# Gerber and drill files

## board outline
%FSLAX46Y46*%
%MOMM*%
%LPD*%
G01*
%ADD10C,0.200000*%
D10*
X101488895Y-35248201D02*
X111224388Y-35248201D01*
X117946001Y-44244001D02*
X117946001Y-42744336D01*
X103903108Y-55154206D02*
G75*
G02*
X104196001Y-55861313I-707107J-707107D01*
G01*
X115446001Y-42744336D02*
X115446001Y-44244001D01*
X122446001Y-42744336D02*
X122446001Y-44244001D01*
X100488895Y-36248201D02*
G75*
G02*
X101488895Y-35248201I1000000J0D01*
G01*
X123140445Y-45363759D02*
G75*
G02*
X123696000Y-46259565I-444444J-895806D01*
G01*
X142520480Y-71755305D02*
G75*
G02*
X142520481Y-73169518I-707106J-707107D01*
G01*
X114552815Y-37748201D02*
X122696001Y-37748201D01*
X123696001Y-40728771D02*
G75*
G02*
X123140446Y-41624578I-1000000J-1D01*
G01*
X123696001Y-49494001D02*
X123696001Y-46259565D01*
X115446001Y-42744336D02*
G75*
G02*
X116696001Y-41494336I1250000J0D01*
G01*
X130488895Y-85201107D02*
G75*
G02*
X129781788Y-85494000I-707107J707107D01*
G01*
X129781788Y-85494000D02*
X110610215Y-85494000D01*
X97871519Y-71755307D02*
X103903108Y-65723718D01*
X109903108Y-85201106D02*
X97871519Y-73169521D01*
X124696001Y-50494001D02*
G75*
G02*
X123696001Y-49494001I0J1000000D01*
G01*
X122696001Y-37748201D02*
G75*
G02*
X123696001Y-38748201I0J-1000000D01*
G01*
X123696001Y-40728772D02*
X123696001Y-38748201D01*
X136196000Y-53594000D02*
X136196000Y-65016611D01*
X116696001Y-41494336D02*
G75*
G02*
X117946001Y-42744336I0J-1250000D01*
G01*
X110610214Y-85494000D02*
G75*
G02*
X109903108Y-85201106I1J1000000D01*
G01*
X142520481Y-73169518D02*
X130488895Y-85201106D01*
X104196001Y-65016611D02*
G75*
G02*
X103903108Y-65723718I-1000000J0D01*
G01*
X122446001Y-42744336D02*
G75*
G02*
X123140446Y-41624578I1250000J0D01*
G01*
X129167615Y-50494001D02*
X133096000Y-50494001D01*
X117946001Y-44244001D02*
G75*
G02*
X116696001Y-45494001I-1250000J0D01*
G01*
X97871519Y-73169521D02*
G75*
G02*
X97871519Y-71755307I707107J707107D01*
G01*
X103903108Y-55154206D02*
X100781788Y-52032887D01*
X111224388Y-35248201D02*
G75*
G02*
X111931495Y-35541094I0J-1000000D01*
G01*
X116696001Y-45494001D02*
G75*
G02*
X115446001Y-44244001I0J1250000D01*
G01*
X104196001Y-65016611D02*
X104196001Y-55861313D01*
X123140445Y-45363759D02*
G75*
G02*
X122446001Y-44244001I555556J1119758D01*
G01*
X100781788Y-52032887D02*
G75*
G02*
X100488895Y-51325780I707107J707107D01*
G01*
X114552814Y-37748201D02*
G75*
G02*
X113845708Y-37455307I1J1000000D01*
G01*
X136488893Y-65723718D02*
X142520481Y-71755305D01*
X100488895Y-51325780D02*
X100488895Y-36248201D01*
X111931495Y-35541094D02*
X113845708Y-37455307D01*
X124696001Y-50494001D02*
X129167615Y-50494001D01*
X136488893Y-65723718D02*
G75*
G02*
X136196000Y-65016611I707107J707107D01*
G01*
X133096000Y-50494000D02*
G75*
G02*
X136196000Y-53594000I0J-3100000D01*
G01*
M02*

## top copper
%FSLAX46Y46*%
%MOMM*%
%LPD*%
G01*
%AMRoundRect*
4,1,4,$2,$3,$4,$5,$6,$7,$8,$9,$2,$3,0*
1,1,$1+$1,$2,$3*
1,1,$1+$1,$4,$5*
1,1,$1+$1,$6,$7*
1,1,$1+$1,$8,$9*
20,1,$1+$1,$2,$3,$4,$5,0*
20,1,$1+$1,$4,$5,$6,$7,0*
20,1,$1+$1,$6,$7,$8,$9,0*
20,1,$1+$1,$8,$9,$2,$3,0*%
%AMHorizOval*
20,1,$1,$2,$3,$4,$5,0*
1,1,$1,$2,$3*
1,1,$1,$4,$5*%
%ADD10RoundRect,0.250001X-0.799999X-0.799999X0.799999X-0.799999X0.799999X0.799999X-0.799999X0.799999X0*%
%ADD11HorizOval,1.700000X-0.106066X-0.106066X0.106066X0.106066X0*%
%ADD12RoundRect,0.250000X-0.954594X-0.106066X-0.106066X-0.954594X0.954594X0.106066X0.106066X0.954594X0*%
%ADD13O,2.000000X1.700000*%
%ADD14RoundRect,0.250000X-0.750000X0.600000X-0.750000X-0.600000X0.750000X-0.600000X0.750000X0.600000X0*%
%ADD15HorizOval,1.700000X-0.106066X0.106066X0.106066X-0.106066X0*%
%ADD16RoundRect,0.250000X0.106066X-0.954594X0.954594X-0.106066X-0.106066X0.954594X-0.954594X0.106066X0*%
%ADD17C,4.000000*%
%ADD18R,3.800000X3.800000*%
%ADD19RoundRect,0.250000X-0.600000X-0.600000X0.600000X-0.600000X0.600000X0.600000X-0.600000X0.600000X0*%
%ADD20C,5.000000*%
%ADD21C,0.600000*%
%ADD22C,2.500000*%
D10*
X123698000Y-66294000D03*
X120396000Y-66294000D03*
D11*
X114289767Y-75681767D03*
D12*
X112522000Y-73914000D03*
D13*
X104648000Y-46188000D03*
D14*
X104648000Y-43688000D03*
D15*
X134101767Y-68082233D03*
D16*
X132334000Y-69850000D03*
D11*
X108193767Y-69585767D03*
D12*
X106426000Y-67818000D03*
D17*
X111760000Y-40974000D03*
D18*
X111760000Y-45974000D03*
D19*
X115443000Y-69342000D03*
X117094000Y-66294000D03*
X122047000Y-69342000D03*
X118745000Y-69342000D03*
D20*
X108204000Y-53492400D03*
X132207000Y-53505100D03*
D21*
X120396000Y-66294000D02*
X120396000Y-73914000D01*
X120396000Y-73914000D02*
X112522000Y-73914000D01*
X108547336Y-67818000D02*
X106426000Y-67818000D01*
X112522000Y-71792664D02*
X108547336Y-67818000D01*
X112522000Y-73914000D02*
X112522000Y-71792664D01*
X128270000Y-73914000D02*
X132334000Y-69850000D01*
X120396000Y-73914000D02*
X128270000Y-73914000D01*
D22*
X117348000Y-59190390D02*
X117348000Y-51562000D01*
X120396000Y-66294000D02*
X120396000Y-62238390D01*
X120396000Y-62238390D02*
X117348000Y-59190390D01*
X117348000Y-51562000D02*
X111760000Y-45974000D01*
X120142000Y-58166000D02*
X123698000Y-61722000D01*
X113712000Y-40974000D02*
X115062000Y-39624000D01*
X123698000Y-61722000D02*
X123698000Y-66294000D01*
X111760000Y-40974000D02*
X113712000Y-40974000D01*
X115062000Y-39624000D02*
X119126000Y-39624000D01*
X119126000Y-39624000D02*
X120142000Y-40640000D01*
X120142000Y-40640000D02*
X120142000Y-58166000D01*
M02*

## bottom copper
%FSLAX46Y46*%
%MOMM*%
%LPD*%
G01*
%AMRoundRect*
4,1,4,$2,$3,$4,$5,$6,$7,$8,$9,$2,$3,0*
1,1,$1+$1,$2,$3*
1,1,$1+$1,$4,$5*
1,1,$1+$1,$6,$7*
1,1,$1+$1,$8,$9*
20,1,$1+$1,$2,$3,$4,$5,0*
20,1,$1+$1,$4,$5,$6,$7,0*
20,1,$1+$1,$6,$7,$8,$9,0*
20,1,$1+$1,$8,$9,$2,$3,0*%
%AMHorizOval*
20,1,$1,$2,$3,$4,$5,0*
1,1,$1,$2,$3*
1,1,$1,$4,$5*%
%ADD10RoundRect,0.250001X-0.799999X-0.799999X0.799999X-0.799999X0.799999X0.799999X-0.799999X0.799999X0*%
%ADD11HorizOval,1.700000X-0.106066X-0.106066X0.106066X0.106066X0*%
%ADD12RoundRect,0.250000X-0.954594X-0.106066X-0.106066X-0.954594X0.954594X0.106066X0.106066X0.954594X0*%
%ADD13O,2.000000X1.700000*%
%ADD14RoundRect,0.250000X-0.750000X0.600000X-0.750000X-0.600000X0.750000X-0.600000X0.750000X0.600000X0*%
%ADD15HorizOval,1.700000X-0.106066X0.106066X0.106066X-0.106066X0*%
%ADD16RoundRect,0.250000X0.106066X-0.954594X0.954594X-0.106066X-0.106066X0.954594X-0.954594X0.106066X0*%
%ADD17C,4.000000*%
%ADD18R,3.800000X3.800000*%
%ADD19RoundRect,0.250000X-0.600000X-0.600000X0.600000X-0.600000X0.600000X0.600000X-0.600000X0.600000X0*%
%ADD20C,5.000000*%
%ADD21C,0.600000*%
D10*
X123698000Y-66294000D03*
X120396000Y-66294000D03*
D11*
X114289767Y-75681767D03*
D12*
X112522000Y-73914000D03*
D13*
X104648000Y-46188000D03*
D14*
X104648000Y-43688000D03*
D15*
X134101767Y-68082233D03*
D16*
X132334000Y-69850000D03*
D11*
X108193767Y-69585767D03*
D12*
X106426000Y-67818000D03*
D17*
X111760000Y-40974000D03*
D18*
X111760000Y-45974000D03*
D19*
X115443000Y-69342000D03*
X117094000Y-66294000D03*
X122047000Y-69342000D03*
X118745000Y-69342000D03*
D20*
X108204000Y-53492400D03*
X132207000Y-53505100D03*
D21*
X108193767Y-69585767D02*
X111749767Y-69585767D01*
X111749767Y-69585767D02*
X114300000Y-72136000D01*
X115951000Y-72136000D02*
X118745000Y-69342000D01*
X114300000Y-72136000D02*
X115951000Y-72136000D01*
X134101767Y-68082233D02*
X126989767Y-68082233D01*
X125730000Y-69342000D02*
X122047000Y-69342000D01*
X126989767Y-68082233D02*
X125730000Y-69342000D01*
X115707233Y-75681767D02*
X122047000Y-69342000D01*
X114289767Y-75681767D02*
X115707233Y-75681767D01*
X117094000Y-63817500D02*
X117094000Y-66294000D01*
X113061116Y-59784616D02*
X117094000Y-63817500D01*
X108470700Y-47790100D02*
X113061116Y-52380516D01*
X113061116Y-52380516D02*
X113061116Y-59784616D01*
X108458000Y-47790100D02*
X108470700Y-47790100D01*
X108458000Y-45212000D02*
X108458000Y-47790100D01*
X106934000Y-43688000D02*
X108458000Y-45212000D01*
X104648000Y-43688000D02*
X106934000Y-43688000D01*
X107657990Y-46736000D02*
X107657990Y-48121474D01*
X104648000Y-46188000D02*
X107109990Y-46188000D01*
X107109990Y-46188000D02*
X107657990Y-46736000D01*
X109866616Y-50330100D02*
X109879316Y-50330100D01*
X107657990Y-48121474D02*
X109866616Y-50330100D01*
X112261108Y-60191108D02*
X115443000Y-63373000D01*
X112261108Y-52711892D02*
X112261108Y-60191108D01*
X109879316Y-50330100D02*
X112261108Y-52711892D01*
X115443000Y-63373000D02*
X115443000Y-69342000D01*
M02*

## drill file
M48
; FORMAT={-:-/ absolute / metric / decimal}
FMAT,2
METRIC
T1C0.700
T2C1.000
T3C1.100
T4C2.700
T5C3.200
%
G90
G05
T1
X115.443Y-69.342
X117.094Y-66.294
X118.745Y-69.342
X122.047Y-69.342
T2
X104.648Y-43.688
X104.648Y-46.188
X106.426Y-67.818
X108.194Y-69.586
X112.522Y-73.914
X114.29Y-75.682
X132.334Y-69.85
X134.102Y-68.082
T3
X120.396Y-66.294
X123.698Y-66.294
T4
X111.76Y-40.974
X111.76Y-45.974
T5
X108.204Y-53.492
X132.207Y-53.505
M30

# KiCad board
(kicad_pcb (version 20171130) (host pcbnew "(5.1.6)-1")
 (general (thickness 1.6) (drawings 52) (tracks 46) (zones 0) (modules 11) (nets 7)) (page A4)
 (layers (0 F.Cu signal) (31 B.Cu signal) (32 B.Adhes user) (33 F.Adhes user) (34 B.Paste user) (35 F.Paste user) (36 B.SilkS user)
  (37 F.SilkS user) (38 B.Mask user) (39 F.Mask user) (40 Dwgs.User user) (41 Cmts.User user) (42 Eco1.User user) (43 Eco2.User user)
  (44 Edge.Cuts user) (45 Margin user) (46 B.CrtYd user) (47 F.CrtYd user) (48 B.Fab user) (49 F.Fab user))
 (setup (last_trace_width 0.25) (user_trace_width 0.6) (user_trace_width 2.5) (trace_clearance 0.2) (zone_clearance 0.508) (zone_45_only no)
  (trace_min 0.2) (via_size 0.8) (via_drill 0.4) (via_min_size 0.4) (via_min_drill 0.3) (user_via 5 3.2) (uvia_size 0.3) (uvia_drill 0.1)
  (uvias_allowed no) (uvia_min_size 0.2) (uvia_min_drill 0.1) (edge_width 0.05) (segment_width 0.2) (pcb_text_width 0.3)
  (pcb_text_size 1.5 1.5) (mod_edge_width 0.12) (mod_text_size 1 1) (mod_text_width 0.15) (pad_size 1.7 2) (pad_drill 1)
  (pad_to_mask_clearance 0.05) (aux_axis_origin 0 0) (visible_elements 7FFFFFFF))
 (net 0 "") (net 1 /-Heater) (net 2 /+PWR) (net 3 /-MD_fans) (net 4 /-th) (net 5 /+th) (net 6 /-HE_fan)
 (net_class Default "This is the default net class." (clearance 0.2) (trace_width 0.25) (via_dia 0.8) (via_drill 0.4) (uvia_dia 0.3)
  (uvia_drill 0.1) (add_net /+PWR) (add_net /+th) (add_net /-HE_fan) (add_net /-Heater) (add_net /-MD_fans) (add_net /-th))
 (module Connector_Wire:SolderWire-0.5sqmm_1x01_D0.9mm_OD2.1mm (layer F.Cu) (at 123.698 66.294)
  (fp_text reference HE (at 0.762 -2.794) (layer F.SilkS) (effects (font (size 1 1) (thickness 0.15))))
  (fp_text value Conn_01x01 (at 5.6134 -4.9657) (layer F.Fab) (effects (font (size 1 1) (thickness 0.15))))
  (pad 1 thru_hole roundrect (at 0 0) (size 2.1 2.1) (drill 1.1) (layers *.Cu *.Mask) (roundrect_rratio 0.119048) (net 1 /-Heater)))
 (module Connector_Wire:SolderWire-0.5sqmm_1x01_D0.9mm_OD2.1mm (layer F.Cu) (at 120.396 66.294)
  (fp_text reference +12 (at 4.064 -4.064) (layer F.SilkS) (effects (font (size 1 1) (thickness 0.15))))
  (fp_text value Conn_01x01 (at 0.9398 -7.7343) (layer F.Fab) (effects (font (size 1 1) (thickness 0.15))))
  (pad 1 thru_hole roundrect (at 0 0) (size 2.1 2.1) (drill 1.1) (layers *.Cu *.Mask) (roundrect_rratio 0.119048) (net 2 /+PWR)))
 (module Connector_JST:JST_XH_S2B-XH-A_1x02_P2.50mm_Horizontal (layer F.Cu) (at 112.522 73.914 315)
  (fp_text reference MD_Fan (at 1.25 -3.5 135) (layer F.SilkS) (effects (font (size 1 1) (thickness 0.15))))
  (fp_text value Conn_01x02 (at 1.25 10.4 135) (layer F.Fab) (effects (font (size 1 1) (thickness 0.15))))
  (pad 2 thru_hole oval (at 2.5 0 315) (size 1.7 2) (drill 1) (layers *.Cu *.Mask) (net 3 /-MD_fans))
  (pad 1 thru_hole roundrect (at 0 0 315) (size 1.7 2) (drill 1) (layers *.Cu *.Mask) (roundrect_rratio 0.147059) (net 2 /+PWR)))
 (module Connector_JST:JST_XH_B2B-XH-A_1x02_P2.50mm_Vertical (layer B.Cu) (at 104.648 43.688 270)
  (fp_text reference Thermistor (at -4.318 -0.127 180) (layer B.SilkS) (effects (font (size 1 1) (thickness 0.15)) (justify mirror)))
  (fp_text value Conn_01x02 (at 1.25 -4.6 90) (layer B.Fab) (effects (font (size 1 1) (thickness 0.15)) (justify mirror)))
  (pad 2 thru_hole oval (at 2.5 0 270) (size 1.7 2) (drill 1) (layers *.Cu *.Mask) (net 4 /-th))
  (pad 1 thru_hole roundrect (at 0 0 270) (size 1.7 2) (drill 1) (layers *.Cu *.Mask) (roundrect_rratio 0.147059) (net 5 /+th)))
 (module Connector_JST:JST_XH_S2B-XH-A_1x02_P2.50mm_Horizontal (layer F.Cu) (at 132.334 69.85 45)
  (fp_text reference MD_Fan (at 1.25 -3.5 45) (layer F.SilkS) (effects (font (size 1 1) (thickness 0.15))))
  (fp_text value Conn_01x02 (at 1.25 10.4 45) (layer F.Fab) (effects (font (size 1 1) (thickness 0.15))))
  (pad 2 thru_hole oval (at 2.5 0 45) (size 1.7 2) (drill 1) (layers *.Cu *.Mask) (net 3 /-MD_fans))
  (pad 1 thru_hole roundrect (at 0 0 45) (size 1.7 2) (drill 1) (layers *.Cu *.Mask) (roundrect_rratio 0.147059) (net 2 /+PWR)))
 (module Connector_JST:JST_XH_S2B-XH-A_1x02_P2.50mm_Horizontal (layer F.Cu) (at 106.426 67.818 315)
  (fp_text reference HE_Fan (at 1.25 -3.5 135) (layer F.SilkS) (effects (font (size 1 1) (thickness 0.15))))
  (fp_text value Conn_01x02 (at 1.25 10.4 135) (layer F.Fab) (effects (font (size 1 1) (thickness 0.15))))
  (pad 2 thru_hole oval (at 2.5 0 315) (size 1.7 2) (drill 1) (layers *.Cu *.Mask) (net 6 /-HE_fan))
  (pad 1 thru_hole roundrect (at 0 0 315) (size 1.7 2) (drill 1) (layers *.Cu *.Mask) (roundrect_rratio 0.147059) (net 2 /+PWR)))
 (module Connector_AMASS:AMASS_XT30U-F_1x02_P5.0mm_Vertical (layer B.Cu) (at 111.76 45.974 90)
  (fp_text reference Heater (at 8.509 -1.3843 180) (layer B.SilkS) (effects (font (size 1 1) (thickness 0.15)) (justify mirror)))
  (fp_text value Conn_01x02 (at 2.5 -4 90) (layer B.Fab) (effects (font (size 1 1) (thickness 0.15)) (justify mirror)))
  (pad 2 thru_hole circle (at 5 0 90) (size 4 4) (drill 2.7) (layers *.Cu *.Mask) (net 1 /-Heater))
  (pad 1 thru_hole rect (at 0 0 90) (size 3.8 3.8) (drill 2.7) (layers *.Cu *.Mask) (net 2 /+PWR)))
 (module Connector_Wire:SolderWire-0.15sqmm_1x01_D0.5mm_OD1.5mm (layer F.Cu) (at 115.443 69.342)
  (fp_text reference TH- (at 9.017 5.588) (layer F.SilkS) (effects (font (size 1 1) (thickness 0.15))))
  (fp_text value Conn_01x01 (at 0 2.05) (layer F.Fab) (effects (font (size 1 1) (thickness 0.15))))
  (pad 1 thru_hole roundrect (at 0 0) (size 1.7 1.7) (drill 0.7) (layers *.Cu *.Mask) (roundrect_rratio 0.147059) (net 4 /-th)))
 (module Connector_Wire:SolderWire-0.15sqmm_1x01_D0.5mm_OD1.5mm (layer F.Cu) (at 117.094 66.294)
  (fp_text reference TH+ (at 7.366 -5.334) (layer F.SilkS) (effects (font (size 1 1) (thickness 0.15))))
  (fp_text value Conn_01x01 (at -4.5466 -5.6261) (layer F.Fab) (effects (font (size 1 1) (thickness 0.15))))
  (pad 1 thru_hole roundrect (at 0 0) (size 1.7 1.7) (drill 0.7) (layers *.Cu *.Mask) (roundrect_rratio 0.147059) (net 5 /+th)))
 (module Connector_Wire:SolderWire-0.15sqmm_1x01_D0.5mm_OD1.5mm (layer F.Cu) (at 122.047 69.342)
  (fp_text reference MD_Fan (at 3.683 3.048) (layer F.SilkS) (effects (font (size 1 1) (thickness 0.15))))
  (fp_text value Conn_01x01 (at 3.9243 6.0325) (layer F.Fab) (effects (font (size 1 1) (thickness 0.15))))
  (pad 1 thru_hole roundrect (at 0 0) (size 1.7 1.7) (drill 0.7) (layers *.Cu *.Mask) (roundrect_rratio 0.147059) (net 3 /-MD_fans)))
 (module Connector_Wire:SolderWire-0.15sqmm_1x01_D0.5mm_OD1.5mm (layer F.Cu) (at 118.745 69.342)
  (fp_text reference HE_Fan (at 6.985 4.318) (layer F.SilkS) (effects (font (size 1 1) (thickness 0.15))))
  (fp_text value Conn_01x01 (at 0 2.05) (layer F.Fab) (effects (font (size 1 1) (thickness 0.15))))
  (pad 1 thru_hole roundrect (at 0 0) (size 1.7 1.7) (drill 0.7) (layers *.Cu *.Mask) (roundrect_rratio 0.147059) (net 6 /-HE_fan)))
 (gr_line (start 101.488895 35.248201) (end 111.224388 35.248201) (layer Edge.Cuts) (width 0.2))
 (gr_line (start 117.946001 44.244001) (end 117.946001 42.744336) (layer Edge.Cuts) (width 0.2))
 (gr_arc (start 103.196001 55.861313) (end 104.196001 55.861313) (angle -45) (layer Edge.Cuts) (width 0.2))
 (gr_line (start 115.446001 42.744336) (end 115.446001 44.244001) (layer Edge.Cuts) (width 0.2))
 (gr_line (start 122.446001 42.744336) (end 122.446001 44.244001) (layer Edge.Cuts) (width 0.2))
 (gr_arc (start 101.488895 36.248201) (end 101.488895 35.248201) (angle -90) (layer Edge.Cuts) (width 0.2))
 (gr_arc (start 122.696001 46.259565) (end 123.696001 46.259565) (angle -63.61220004) (layer Edge.Cuts) (width 0.2))
 (gr_arc (start 141.813374 72.462412) (end 142.520481 73.169518) (angle -89.99999715) (layer Edge.Cuts) (width 0.2))
 (gr_line (start 114.552815 37.748201) (end 122.696001 37.748201) (layer Edge.Cuts) (width 0.2))
 (gr_arc (start 122.696001 40.728772) (end 123.140446 41.624578) (angle -63.61220004) (layer Edge.Cuts) (width 0.2))
 (gr_line (start 123.696001 49.494001) (end 123.696001 46.259565) (layer Edge.Cuts) (width 0.2))
 (gr_arc (start 116.696001 42.744336) (end 116.696001 41.494336) (angle -90) (layer Edge.Cuts) (width 0.2))
 (gr_arc (start 129.781788 84.494) (end 129.781788 85.494) (angle -45.00000244) (layer Edge.Cuts) (width 0.2))
 (gr_line (start 129.781788 85.494) (end 110.610215 85.494) (layer Edge.Cuts) (width 0.2))
 (gr_line (start 97.871519 71.755307) (end 103.903108 65.723718) (layer Edge.Cuts) (width 0.2))
 (gr_line (start 109.903108 85.201106) (end 97.871519 73.169521) (layer Edge.Cuts) (width 0.2))
 (gr_arc (start 124.696001 49.494001) (end 123.696001 49.494001) (angle -90) (layer Edge.Cuts) (width 0.2))
 (gr_arc (start 122.696001 38.748201) (end 123.696001 38.748201) (angle -90) (layer Edge.Cuts) (width 0.2))
 (gr_line (start 123.696001 40.728772) (end 123.696001 38.748201) (layer Edge.Cuts) (width 0.2))
 (gr_line (start 136.196 53.594) (end 136.196 65.016611) (layer Edge.Cuts) (width 0.2))
 (gr_arc (start 116.696001 42.744336) (end 117.946001 42.744336) (angle -90) (layer Edge.Cuts) (width 0.2))
 (gr_arc (start 110.610215 84.494) (end 109.903108 85.201106) (angle -44.99999269) (layer Edge.Cuts) (width 0.2))
 (gr_line (start 142.520481 73.169518) (end 130.488895 85.201106) (layer Edge.Cuts) (width 0.2))
 (gr_arc (start 103.196001 65.016611) (end 103.903108 65.723718) (angle -44.99999916) (layer Edge.Cuts) (width 0.2))
 (gr_arc (start 123.696001 42.744336) (end 123.140446 41.624578) (angle -63.61220004) (layer Edge.Cuts) (width 0.2))
 (gr_line (start 129.167615 50.494001) (end 133.096 50.494001) (layer Edge.Cuts) (width 0.2))
 (gr_arc (start 116.696001 44.244001) (end 116.696001 45.494001) (angle -90) (layer Edge.Cuts) (width 0.2))
 (gr_arc (start 98.578626 72.462414) (end 97.871519 71.755307) (angle -90.00000647) (layer Edge.Cuts) (width 0.2))
 (gr_line (start 103.903108 55.154206) (end 100.781788 52.032887) (layer Edge.Cuts) (width 0.2))
 (gr_arc (start 111.224388 36.248201) (end 111.931495 35.541094) (angle -45) (layer Edge.Cuts) (width 0.2))
 (gr_arc (start 116.696001 44.244001) (end 115.446001 44.244001) (angle -90) (layer Edge.Cuts) (width 0.2))
 (gr_line (start 104.196001 65.016611) (end 104.196001 55.861313) (layer Edge.Cuts) (width 0.2))
 (gr_arc (start 123.696001 44.244001) (end 122.446001 44.244001) (angle -63.61220004) (layer Edge.Cuts) (width 0.2))
 (gr_arc (start 101.488895 51.32578) (end 100.488895 51.32578) (angle -45) (layer Edge.Cuts) (width 0.2))
 (gr_arc (start 114.552815 36.748201) (end 113.845708 37.455307) (angle -45) (layer Edge.Cuts) (width 0.2))
 (gr_line (start 136.488893 65.723718) (end 142.520481 71.755305) (layer Edge.Cuts) (width 0.2))
 (gr_line (start 100.488895 51.32578) (end 100.488895 36.248201) (layer Edge.Cuts) (width 0.2))
 (gr_line (start 111.931495 35.541094) (end 113.845708 37.455307) (layer Edge.Cuts) (width 0.2))
 (gr_line (start 124.696001 50.494001) (end 129.167615 50.494001) (layer Edge.Cuts) (width 0.2))
 (gr_arc (start 137.196 65.016611) (end 136.196 65.016611) (angle -44.99999958) (layer Edge.Cuts) (width 0.2))
 (gr_arc (start 133.096 53.594) (end 136.196 53.594) (angle -90) (layer Edge.Cuts) (width 0.2))
 (via (at 108.204 53.4924) (size 5) (drill 3.2) (layers F.Cu B.Cu) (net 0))
 (via (at 132.207 53.5051) (size 5) (drill 3.2) (layers F.Cu B.Cu) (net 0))
 (segment (start 120.396 66.294) (end 120.396 73.914) (width 0.6) (layer F.Cu) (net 2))
 (segment (start 120.396 73.914) (end 112.522 73.914) (width 0.6) (layer F.Cu) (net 2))
 (segment (start 108.547336 67.818) (end 106.426 67.818) (width 0.6) (layer F.Cu) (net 2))
 (segment (start 112.522 71.792664) (end 108.547336 67.818) (width 0.6) (layer F.Cu) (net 2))
 (segment (start 112.522 73.914) (end 112.522 71.792664) (width 0.6) (layer F.Cu) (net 2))
 (segment (start 128.27 73.914) (end 132.334 69.85) (width 0.6) (layer F.Cu) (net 2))
 (segment (start 120.396 73.914) (end 128.27 73.914) (width 0.6) (layer F.Cu) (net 2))
 (segment (start 117.348 59.19039) (end 117.348 51.562) (width 2.5) (layer F.Cu) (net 2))
 (segment (start 120.396 66.294) (end 120.396 62.23839) (width 2.5) (layer F.Cu) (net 2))
 (segment (start 120.396 62.23839) (end 117.348 59.19039) (width 2.5) (layer F.Cu) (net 2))
 (segment (start 117.348 51.562) (end 111.76 45.974) (width 2.5) (layer F.Cu) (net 2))
 (segment (start 120.142 58.166) (end 123.698 61.722) (width 2.5) (layer F.Cu) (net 1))
 (segment (start 113.712 40.974) (end 115.062 39.624) (width 2.5) (layer F.Cu) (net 1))
 (segment (start 123.698 61.722) (end 123.698 66.294) (width 2.5) (layer F.Cu) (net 1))
 (segment (start 111.76 40.974) (end 113.712 40.974) (width 2.5) (layer F.Cu) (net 1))
 (segment (start 115.062 39.624) (end 119.126 39.624) (width 2.5) (layer F.Cu) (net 1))
 (segment (start 119.126 39.624) (end 120.142 40.64) (width 2.5) (layer F.Cu) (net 1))
 (segment (start 120.142 40.64) (end 120.142 58.166) (width 2.5) (layer F.Cu) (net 1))
 (segment (start 108.193767 69.585767) (end 111.749767 69.585767) (width 0.6) (layer B.Cu) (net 6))
 (segment (start 111.749767 69.585767) (end 114.3 72.136) (width 0.6) (layer B.Cu) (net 6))
 (segment (start 115.951 72.136) (end 118.745 69.342) (width 0.6) (layer B.Cu) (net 6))
 (segment (start 114.3 72.136) (end 115.951 72.136) (width 0.6) (layer B.Cu) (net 6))
 (segment (start 134.101767 68.082233) (end 126.989767 68.082233) (width 0.6) (layer B.Cu) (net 3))
 (segment (start 125.73 69.342) (end 122.047 69.342) (width 0.6) (layer B.Cu) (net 3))
 (segment (start 126.989767 68.082233) (end 125.73 69.342) (width 0.6) (layer B.Cu) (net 3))
 (segment (start 115.707233 75.681767) (end 122.047 69.342) (width 0.6) (layer B.Cu) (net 3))
 (segment (start 114.289767 75.681767) (end 115.707233 75.681767) (width 0.6) (layer B.Cu) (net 3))
 (segment (start 117.094 63.8175) (end 117.094 66.294) (width 0.6) (layer B.Cu) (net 5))
 (segment (start 113.061116 59.784616) (end 117.094 63.8175) (width 0.6) (layer B.Cu) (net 5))
 (segment (start 108.4707 47.7901) (end 113.061116 52.380516) (width 0.6) (layer B.Cu) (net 5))
 (segment (start 113.061116 52.380516) (end 113.061116 59.784616) (width 0.6) (layer B.Cu) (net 5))
 (segment (start 108.458 47.7901) (end 108.4707 47.7901) (width 0.6) (layer B.Cu) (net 5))
 (segment (start 108.458 45.212) (end 108.458 47.7901) (width 0.6) (layer B.Cu) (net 5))
 (segment (start 106.934 43.688) (end 108.458 45.212) (width 0.6) (layer B.Cu) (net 5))
 (segment (start 104.648 43.688) (end 106.934 43.688) (width 0.6) (layer B.Cu) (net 5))
 (segment (start 107.65799 46.736) (end 107.65799 48.121474) (width 0.6) (layer B.Cu) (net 4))
 (segment (start 104.648 46.188) (end 107.10999 46.188) (width 0.6) (layer B.Cu) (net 4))
 (segment (start 107.10999 46.188) (end 107.65799 46.736) (width 0.6) (layer B.Cu) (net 4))
 (segment (start 109.866616 50.3301) (end 109.879316 50.3301) (width 0.6) (layer B.Cu) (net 4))
 (segment (start 107.65799 48.121474) (end 109.866616 50.3301) (width 0.6) (layer B.Cu) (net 4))
 (segment (start 112.261108 60.191108) (end 115.443 63.373) (width 0.6) (layer B.Cu) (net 4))
 (segment (start 112.261108 52.711892) (end 112.261108 60.191108) (width 0.6) (layer B.Cu) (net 4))
 (segment (start 109.879316 50.3301) (end 112.261108 52.711892) (width 0.6) (layer B.Cu) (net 4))
 (segment (start 115.443 63.373) (end 115.443 69.342) (width 0.6) (layer B.Cu) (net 4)))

